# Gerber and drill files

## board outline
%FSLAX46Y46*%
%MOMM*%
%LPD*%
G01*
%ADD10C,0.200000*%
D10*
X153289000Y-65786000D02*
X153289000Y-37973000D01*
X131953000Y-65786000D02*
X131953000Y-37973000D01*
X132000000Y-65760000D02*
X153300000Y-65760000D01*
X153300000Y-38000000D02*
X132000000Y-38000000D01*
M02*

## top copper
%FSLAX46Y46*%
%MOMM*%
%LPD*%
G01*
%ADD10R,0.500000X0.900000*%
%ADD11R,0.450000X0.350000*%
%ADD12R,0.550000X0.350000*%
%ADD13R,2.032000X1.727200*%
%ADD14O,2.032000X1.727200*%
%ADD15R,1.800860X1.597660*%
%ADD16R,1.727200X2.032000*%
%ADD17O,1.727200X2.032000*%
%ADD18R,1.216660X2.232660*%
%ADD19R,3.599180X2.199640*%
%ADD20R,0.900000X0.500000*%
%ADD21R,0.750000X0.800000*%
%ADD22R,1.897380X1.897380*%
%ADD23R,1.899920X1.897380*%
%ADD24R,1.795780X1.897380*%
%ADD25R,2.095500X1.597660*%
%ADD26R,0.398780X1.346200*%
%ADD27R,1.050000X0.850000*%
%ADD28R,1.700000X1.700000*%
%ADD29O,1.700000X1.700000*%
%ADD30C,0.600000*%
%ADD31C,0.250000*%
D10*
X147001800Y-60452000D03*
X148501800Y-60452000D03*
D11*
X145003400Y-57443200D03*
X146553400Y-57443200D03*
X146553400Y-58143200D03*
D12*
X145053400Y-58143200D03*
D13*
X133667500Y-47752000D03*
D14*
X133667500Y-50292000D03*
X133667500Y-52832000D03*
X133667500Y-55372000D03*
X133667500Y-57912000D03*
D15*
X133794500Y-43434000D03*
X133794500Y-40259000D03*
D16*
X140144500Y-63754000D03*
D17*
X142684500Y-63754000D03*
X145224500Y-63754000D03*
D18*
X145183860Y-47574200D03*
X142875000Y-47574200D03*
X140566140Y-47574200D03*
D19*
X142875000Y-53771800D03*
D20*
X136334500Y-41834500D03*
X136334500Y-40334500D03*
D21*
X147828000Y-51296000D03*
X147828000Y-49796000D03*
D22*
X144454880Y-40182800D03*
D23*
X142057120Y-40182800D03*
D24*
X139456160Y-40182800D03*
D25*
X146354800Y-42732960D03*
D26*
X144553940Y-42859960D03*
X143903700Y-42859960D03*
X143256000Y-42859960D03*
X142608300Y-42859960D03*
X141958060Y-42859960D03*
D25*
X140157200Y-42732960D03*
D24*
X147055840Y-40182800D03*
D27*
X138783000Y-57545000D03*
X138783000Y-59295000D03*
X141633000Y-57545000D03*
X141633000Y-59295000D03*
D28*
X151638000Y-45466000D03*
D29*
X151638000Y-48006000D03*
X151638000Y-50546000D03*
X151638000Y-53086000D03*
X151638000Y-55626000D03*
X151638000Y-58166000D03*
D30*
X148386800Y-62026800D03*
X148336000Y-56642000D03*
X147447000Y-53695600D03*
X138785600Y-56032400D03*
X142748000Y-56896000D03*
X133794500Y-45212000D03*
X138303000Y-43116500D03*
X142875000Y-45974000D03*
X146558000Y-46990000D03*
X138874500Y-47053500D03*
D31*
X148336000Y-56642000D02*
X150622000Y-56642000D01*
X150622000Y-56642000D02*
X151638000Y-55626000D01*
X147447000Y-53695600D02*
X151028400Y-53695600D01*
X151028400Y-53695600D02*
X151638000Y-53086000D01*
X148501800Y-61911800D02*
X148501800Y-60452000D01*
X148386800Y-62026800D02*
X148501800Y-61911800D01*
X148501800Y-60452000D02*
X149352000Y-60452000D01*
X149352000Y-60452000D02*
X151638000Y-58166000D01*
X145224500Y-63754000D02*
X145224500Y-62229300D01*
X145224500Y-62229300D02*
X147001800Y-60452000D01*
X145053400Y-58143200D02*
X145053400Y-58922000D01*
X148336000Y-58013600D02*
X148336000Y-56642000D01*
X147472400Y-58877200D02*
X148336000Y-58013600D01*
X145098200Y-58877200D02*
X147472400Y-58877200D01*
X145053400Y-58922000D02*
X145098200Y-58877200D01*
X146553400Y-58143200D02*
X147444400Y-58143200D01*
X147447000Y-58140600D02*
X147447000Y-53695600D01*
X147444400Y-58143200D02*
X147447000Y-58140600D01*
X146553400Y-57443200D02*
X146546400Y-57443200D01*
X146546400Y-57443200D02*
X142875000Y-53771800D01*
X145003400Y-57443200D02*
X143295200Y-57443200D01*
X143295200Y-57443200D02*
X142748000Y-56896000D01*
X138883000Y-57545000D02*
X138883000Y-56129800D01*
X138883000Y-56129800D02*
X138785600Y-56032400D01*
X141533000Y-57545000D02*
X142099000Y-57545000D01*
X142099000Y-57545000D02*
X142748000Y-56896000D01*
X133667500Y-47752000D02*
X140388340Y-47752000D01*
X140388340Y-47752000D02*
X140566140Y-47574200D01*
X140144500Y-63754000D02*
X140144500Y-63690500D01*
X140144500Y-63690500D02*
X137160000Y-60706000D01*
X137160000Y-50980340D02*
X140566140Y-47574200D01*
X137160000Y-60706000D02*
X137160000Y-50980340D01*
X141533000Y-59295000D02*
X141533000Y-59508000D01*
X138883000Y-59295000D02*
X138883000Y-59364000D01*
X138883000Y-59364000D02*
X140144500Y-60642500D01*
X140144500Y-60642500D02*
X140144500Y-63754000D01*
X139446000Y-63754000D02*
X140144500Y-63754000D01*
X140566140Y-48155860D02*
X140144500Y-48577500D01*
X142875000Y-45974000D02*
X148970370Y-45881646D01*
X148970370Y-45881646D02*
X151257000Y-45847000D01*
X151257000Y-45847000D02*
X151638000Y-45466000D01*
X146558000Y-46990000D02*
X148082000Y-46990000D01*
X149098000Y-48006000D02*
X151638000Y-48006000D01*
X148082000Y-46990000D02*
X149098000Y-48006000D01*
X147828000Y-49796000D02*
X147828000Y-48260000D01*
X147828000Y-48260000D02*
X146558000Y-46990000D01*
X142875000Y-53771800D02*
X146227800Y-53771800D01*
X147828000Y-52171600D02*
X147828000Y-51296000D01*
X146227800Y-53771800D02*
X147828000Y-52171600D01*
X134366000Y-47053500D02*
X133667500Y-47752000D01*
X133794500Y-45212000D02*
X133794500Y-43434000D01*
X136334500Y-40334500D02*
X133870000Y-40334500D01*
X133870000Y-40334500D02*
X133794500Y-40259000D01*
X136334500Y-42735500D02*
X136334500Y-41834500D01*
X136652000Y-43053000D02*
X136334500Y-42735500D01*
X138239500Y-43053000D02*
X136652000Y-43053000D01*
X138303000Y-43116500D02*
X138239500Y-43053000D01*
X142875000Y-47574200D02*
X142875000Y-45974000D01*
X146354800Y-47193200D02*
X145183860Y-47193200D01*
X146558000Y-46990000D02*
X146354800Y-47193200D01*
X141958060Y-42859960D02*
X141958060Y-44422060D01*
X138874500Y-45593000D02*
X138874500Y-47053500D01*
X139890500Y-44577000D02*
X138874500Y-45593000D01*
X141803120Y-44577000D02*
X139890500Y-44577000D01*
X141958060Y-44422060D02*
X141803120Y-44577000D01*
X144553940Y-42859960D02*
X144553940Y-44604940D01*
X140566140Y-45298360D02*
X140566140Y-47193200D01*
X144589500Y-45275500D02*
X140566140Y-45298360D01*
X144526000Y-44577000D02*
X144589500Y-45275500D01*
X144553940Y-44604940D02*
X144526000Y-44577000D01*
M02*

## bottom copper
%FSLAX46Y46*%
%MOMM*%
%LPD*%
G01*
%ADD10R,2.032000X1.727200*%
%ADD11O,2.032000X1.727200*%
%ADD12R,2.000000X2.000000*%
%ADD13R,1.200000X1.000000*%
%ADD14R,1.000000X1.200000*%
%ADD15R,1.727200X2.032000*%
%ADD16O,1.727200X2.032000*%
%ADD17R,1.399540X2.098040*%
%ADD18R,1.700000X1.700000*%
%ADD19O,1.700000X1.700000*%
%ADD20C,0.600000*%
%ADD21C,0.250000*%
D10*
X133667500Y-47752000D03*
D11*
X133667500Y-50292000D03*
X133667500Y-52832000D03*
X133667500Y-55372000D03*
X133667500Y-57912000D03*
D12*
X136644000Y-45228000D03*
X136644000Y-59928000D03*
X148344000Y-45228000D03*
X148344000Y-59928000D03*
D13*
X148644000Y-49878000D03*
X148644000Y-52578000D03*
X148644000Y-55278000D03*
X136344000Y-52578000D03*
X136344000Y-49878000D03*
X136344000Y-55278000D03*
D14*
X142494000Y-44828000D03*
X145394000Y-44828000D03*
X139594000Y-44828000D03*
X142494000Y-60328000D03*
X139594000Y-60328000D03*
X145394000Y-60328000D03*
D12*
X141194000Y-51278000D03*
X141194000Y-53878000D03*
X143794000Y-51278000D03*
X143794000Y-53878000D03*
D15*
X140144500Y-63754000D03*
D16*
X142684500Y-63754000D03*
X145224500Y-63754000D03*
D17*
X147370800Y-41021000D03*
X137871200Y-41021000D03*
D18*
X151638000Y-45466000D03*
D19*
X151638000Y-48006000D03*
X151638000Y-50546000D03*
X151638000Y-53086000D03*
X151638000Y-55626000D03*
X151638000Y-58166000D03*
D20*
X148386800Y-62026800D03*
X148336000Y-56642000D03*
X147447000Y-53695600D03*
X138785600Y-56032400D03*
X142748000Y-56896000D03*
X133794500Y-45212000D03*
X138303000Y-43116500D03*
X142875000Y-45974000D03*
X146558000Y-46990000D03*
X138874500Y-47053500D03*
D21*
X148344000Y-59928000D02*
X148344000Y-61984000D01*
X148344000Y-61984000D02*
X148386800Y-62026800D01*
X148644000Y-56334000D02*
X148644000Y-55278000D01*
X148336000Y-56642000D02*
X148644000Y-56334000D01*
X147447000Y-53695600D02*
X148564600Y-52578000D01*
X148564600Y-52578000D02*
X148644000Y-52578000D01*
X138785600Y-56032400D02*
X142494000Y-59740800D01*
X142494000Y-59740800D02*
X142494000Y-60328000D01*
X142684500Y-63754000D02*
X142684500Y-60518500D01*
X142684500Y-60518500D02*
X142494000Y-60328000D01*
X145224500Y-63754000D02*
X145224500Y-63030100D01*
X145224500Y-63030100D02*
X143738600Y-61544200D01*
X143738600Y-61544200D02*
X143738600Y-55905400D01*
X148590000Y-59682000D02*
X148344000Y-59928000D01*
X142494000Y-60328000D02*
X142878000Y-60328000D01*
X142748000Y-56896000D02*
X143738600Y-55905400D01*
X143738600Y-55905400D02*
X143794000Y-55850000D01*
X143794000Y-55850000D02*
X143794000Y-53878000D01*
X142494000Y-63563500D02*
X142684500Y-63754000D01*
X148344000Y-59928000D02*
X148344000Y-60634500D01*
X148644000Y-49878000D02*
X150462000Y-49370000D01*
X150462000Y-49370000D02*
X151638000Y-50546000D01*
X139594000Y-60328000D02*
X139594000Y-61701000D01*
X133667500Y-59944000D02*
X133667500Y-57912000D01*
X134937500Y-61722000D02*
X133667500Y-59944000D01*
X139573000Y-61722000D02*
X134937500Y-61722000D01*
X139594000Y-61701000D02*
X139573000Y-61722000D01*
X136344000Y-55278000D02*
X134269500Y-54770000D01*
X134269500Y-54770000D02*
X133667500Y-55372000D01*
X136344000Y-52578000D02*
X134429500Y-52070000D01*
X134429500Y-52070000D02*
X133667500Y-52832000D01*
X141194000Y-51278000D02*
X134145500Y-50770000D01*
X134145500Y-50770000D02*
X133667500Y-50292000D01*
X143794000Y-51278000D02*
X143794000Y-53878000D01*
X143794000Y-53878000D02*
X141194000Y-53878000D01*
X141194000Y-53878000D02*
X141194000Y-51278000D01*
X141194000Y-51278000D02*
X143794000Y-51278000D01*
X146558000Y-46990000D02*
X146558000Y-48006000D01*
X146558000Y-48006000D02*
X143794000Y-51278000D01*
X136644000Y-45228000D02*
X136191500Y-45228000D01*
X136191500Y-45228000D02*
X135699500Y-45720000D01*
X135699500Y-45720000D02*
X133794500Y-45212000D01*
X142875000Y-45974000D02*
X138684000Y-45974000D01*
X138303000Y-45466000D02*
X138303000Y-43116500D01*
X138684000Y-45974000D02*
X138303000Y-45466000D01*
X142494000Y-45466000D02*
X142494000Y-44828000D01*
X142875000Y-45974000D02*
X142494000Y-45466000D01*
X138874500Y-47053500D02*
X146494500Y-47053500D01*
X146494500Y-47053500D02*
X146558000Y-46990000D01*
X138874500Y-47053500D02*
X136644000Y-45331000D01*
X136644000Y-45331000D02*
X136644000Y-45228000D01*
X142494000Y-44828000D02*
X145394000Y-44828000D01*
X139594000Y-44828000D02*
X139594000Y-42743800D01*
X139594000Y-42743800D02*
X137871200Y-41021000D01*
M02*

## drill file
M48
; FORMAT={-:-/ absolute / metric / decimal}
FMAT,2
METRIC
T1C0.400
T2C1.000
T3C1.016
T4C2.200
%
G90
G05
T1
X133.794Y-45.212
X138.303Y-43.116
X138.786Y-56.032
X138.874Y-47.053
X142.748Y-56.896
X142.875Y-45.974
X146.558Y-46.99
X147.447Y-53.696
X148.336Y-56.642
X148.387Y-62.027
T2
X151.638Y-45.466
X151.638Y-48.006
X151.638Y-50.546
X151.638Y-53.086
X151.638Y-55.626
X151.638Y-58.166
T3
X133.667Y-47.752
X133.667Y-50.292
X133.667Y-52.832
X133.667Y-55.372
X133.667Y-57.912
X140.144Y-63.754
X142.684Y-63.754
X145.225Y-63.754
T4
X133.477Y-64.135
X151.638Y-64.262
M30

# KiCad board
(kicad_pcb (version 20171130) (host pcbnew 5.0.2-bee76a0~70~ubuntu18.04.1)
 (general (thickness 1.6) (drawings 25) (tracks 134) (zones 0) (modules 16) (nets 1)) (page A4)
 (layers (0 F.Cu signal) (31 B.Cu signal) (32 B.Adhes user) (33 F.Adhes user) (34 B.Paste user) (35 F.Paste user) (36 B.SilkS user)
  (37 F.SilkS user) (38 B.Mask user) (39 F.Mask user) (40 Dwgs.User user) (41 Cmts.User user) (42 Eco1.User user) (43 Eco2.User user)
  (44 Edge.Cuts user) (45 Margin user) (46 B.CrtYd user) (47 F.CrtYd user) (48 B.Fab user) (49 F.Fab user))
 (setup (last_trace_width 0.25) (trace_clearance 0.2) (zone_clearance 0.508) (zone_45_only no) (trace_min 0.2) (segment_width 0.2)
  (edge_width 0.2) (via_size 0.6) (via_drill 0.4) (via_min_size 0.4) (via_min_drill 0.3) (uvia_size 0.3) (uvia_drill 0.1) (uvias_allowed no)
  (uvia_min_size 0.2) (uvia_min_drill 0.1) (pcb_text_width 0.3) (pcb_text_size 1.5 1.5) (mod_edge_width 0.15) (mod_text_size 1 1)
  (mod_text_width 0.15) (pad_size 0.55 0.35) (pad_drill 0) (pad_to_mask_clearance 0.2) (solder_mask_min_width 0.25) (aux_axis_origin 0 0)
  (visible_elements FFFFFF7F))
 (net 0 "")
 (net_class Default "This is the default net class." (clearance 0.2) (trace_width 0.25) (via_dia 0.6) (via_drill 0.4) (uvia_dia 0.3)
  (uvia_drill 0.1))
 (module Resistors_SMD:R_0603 (layer F.Cu) (at 147.7518 60.452)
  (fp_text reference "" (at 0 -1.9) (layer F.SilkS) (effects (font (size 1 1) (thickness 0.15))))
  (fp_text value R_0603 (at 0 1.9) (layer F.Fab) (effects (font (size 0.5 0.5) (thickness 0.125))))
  (pad 1 smd rect (at -0.75 0) (size 0.5 0.9) (layers F.Cu F.Paste F.Mask))
  (pad 2 smd rect (at 0.75 0) (size 0.5 0.9) (layers F.Cu F.Paste F.Mask)))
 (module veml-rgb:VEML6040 (layer F.Cu) (at 145.9484 56.7182)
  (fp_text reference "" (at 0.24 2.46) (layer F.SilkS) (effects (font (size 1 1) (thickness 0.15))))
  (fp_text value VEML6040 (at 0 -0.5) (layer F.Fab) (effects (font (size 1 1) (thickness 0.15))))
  (pad GND smd rect (at -0.945 0.725) (size 0.45 0.35) (layers F.Cu F.Paste F.Mask))
  (pad +V smd rect (at 0.605 0.725) (size 0.45 0.35) (layers F.Cu F.Paste F.Mask))
  (pad 3 smd rect (at 0.605 1.425) (size 0.45 0.35) (layers F.Cu F.Paste F.Mask))
  (pad 2 smd rect (at -0.895 1.425) (size 0.55 0.35) (layers F.Cu F.Paste F.Mask)))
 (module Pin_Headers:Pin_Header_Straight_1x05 (layer F.Cu) (at 133.6675 47.752)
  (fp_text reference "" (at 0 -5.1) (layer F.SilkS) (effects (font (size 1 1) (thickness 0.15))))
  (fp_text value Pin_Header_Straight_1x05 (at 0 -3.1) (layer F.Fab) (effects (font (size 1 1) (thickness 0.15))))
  (pad 1 thru_hole rect (at 0 0) (size 2.032 1.7272) (drill 1.016) (layers *.Cu *.Mask F.SilkS))
  (pad 2 thru_hole oval (at 0 2.54) (size 2.032 1.7272) (drill 1.016) (layers *.Cu *.Mask F.SilkS))
  (pad 3 thru_hole oval (at 0 5.08) (size 2.032 1.7272) (drill 1.016) (layers *.Cu *.Mask F.SilkS))
  (pad 4 thru_hole oval (at 0 7.62) (size 2.032 1.7272) (drill 1.016) (layers *.Cu *.Mask F.SilkS))
  (pad 5 thru_hole oval (at 0 10.16) (size 2.032 1.7272) (drill 1.016) (layers *.Cu *.Mask F.SilkS)))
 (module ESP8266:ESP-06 (layer B.Cu) (at 142.494 52.578 270)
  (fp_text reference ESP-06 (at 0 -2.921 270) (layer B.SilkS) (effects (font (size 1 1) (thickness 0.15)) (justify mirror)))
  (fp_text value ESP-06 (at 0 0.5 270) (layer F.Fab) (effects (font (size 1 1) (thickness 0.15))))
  (pad GND smd rect (at -7.35 5.85 270) (size 2 2) (layers B.Cu B.Paste B.Mask))
  (pad GP5 smd rect (at 7.35 5.85 270) (size 2 2) (layers B.Cu B.Paste B.Mask))
  (pad GP16 smd rect (at -7.35 -5.85 270) (size 2 2) (layers B.Cu B.Paste B.Mask))
  (pad GP15 smd rect (at 7.35 -5.85 270) (size 2 2) (layers B.Cu B.Paste B.Mask))
  (pad GP14 smd rect (at -2.7 -6.15 270) (size 1 1.2) (layers B.Cu B.Paste B.Mask))
  (pad GP12 smd rect (at 0 -6.15 270) (size 1 1.2) (layers B.Cu B.Paste B.Mask))
  (pad GP13 smd rect (at 2.7 -6.15 270) (size 1 1.2) (layers B.Cu B.Paste B.Mask))
  (pad TX smd rect (at 0 6.15 270) (size 1 1.2) (layers B.Cu B.Paste B.Mask))
  (pad RST smd rect (at -2.7 6.15 270) (size 1 1.2) (layers B.Cu B.Paste B.Mask))
  (pad RX smd rect (at 2.7 6.15 270) (size 1 1.2) (layers B.Cu B.Paste B.Mask))
  (pad 3.3 smd rect (at -7.75 0 270) (size 1.2 1) (layers B.Cu B.Paste B.Mask))
  (pad CHPD smd rect (at -7.75 -2.9 270) (size 1.2 1) (layers B.Cu B.Paste B.Mask))
  (pad ANT smd rect (at -7.75 2.9 270) (size 1.2 1) (layers B.Cu B.Paste B.Mask))
  (pad GP2 smd rect (at 7.75 0 270) (size 1.2 1) (layers B.Cu B.Paste B.Mask))
  (pad GP0 smd rect (at 7.75 2.9 270) (size 1.2 1) (layers B.Cu B.Paste B.Mask))
  (pad GP4 smd rect (at 7.75 -2.9 270) (size 1.2 1) (layers B.Cu B.Paste B.Mask))
  (pad GND smd rect (at -1.3 1.3 270) (size 2 2) (layers B.Cu B.Paste B.Mask))
  (pad GND smd rect (at 1.3 1.3 270) (size 2 2) (layers B.Cu B.Paste B.Mask))
  (pad GND smd rect (at -1.3 -1.3 270) (size 2 2) (layers B.Cu B.Paste B.Mask))
  (pad GND smd rect (at 1.3 -1.3 270) (size 2 2) (layers B.Cu B.Paste B.Mask)))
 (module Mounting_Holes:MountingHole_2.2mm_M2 (layer F.Cu) (at 133.477 64.135)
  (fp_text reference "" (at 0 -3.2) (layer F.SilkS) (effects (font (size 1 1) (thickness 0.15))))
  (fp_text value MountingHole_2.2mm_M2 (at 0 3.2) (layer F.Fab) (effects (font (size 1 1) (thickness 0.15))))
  (pad 1 np_thru_hole circle (at 0 0) (size 2.2 2.2) (drill 2.2) (layers *.Cu *.Mask F.SilkS)))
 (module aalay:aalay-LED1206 (layer F.Cu) (at 133.7945 41.8465 90)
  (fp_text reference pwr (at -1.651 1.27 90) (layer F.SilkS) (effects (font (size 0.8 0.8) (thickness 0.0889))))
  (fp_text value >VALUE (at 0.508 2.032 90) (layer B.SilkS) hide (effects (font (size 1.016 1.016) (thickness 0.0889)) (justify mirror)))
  (pad A smd rect (at -1.5875 0 90) (size 1.59766 1.80086) (layers F.Cu F.Paste F.Mask))
  (pad K smd rect (at 1.5875 0 90) (size 1.59766 1.80086) (layers F.Cu F.Paste F.Mask)))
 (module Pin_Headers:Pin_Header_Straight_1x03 (layer F.Cu) (at 140.1445 63.754 90)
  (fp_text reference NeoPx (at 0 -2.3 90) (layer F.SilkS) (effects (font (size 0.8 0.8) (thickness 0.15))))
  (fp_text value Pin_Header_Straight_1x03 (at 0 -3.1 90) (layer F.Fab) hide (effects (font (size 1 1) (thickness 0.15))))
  (pad 1 thru_hole rect (at 0 0 90) (size 2.032 1.7272) (drill 1.016) (layers *.Cu *.Mask F.SilkS))
  (pad 2 thru_hole oval (at 0 2.54 90) (size 2.032 1.7272) (drill 1.016) (layers *.Cu *.Mask F.SilkS))
  (pad 3 thru_hole oval (at 0 5.08 90) (size 2.032 1.7272) (drill 1.016) (layers *.Cu *.Mask F.SilkS)))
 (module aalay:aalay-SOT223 (layer F.Cu) (at 142.875 50.673 180)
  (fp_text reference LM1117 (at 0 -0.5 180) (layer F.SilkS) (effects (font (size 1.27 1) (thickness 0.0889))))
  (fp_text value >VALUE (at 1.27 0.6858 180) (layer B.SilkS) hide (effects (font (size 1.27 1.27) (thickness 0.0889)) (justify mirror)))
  (pad GND smd rect (at -2.30886 3.0988 180) (size 1.21666 2.23266) (layers F.Cu F.Paste F.Mask))
  (pad OUT smd rect (at 0 3.0988 180) (size 1.21666 2.23266) (layers F.Cu F.Paste F.Mask))
  (pad IN smd rect (at 2.30886 3.0988 180) (size 1.21666 2.23266) (layers F.Cu F.Paste F.Mask))
  (pad OUT smd rect (at 0 -3.0988 180) (size 3.59918 2.19964) (layers F.Cu F.Paste F.Mask)))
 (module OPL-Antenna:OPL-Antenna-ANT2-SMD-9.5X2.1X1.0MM (layer B.Cu) (at 142.621 41.021 180)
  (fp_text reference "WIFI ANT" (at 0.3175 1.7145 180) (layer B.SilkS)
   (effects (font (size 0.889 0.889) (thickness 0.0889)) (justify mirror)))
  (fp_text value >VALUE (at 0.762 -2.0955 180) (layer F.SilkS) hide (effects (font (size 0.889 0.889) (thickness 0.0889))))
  (pad 1 smd rect (at -4.7498 0 180) (size 1.39954 2.09804) (layers B.Cu B.Paste B.Mask))
  (pad 2 smd rect (at 4.7498 0 180) (size 1.39954 2.09804) (layers B.Cu B.Paste B.Mask)))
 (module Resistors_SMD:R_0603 (layer F.Cu) (at 136.3345 41.0845 90)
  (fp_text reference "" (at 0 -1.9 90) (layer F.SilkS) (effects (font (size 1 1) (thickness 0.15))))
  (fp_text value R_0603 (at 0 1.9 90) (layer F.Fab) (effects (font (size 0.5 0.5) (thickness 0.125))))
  (pad 1 smd rect (at -0.75 0 90) (size 0.5 0.9) (layers F.Cu F.Paste F.Mask))
  (pad 2 smd rect (at 0.75 0 90) (size 0.5 0.9) (layers F.Cu F.Paste F.Mask)))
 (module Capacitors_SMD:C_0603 (layer F.Cu) (at 147.828 50.546 90)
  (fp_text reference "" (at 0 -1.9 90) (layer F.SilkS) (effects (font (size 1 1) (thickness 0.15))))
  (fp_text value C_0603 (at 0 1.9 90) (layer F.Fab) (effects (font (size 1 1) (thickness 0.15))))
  (pad 1 smd rect (at -0.75 0 90) (size 0.8 0.75) (layers F.Cu F.Paste F.Mask))
  (pad 2 smd rect (at 0.75 0 90) (size 0.8 0.75) (layers F.Cu F.Paste F.Mask)))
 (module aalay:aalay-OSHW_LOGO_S (layer F.Cu) (at 150.622 39.878)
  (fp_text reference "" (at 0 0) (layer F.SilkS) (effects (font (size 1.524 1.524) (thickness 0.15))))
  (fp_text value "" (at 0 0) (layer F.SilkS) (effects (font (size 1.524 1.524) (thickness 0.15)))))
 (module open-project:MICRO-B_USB (layer F.Cu) (at 143.256 38.735 180)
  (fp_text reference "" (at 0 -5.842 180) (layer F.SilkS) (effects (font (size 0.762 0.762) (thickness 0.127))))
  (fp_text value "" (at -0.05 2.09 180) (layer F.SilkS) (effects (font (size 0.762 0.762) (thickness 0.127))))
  (pad "" smd rect (at -1.19888 -1.4478 180) (size 1.89738 1.89738) (layers F.Cu F.Paste F.Mask))
  (pad "" smd rect (at 1.19888 -1.4478 180) (size 1.89992 1.89738) (layers F.Cu F.Paste F.Mask))
  (pad "" smd rect (at 3.79984 -1.4478 180) (size 1.79578 1.89738) (layers F.Cu F.Paste F.Mask))
  (pad "" smd rect (at -3.0988 -3.99796 180) (size 2.0955 1.59766) (layers F.Cu F.Paste F.Mask))
  (pad +5 smd rect (at -1.29794 -4.12496 180) (size 0.39878 1.3462) (layers F.Cu F.Paste F.Mask) (clearance 0.2032))
  (pad 2 smd rect (at -0.6477 -4.12496 180) (size 0.39878 1.3462) (layers F.Cu F.Paste F.Mask) (clearance 0.2032))
  (pad 3 smd rect (at 0 -4.12496 180) (size 0.39878 1.3462) (layers F.Cu F.Paste F.Mask) (clearance 0.2032))
  (pad 4 smd rect (at 0.6477 -4.12496 180) (size 0.39878 1.3462) (layers F.Cu F.Paste F.Mask) (clearance 0.2032))
  (pad GND smd rect (at 1.29794 -4.12496 180) (size 0.39878 1.3462) (layers F.Cu F.Paste F.Mask) (clearance 0.2032))
  (pad "" smd rect (at 3.0988 -3.99796 180) (size 2.0955 1.59766) (layers F.Cu F.Paste F.Mask))
  (pad "" smd rect (at -3.79984 -1.4478 180) (size 1.79578 1.89738) (layers F.Cu F.Paste F.Mask)))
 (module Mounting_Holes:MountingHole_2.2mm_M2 (layer F.Cu) (at 151.638 64.262)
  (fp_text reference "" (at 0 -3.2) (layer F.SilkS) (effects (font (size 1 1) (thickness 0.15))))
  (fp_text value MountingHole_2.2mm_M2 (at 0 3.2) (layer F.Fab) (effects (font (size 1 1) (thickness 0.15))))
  (pad 1 np_thru_hole circle (at 0 0) (size 2.2 2.2) (drill 2.2) (layers *.Cu *.Mask F.SilkS)))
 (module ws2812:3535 (layer F.Cu) (at 140.208 58.42 180)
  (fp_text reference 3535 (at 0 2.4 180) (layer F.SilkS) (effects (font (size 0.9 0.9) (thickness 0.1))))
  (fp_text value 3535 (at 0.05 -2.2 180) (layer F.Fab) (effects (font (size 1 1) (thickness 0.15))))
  (pad IN smd rect (at 1.325 0.875 180) (size 1.05 0.85) (drill (offset 0.1 0)) (layers F.Cu F.Paste F.Mask))
  (pad VDD smd rect (at 1.325 -0.875 180) (size 1.05 0.85) (drill (offset 0.1 0)) (layers F.Cu F.Paste F.Mask))
  (pad GND smd rect (at -1.325 0.875 180) (size 1.05 0.85) (drill (offset -0.1 0)) (layers F.Cu F.Paste F.Mask))
  (pad OUT smd rect (at -1.325 -0.875 180) (size 1.05 0.85) (drill (offset -0.1 0)) (layers F.Cu F.Paste F.Mask)))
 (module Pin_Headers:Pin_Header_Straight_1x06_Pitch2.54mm (layer F.Cu) (at 151.638 45.466)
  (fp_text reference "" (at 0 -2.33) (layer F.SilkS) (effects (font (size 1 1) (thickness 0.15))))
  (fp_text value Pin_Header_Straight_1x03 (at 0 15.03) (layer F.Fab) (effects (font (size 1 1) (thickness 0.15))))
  (pad 1 thru_hole rect (at 0 0) (size 1.7 1.7) (drill 1) (layers *.Cu *.Mask))
  (pad 2 thru_hole oval (at 0 2.54) (size 1.7 1.7) (drill 1) (layers *.Cu *.Mask))
  (pad 3 thru_hole oval (at 0 5.08) (size 1.7 1.7) (drill 1) (layers *.Cu *.Mask))
  (pad 4 thru_hole oval (at 0 7.62) (size 1.7 1.7) (drill 1) (layers *.Cu *.Mask))
  (pad 5 thru_hole oval (at 0 10.16) (size 1.7 1.7) (drill 1) (layers *.Cu *.Mask))
  (pad 6 thru_hole oval (at 0 12.7) (size 1.7 1.7) (drill 1) (layers *.Cu *.Mask)))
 (gr_line (start 153.289 65.786) (end 153.289 37.973) (angle 90) (layer Edge.Cuts) (width 0.2))
 (gr_line (start 131.953 65.786) (end 131.953 37.973) (angle 90) (layer Edge.Cuts) (width 0.2))
 (gr_line (start 132 65.76) (end 153.3 65.76) (angle 90) (layer Edge.Cuts) (width 0.2))
 (gr_line (start 153.3 38) (end 132 38) (angle 90) (layer Edge.Cuts) (width 0.2))
 (segment (start 148.336 56.642) (end 150.622 56.642) (width 0.25) (layer F.Cu) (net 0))
 (segment (start 150.622 56.642) (end 151.638 55.626) (width 0.25) (layer F.Cu) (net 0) (status 800000))
 (segment (start 147.447 53.6956) (end 151.0284 53.6956) (width 0.25) (layer F.Cu) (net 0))
 (segment (start 151.0284 53.6956) (end 151.638 53.086) (width 0.25) (layer F.Cu) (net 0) (status 800000))
 (segment (start 148.344 59.928) (end 148.344 61.984) (width 0.25) (layer B.Cu) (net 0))
 (segment (start 148.5018 61.9118) (end 148.5018 60.452) (width 0.25) (layer F.Cu) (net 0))
 (segment (start 148.3868 62.0268) (end 148.5018 61.9118) (width 0.25) (layer F.Cu) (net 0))
 (via (at 148.3868 62.0268) (size 0.6) (drill 0.4) (layers F.Cu B.Cu) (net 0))
 (segment (start 148.344 61.984) (end 148.3868 62.0268) (width 0.25) (layer B.Cu) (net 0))
 (segment (start 148.5018 60.452) (end 149.352 60.452) (width 0.25) (layer F.Cu) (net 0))
 (segment (start 149.352 60.452) (end 151.638 58.166) (width 0.25) (layer F.Cu) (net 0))
 (segment (start 145.2245 63.754) (end 145.2245 62.2293) (width 0.25) (layer F.Cu) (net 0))
 (segment (start 145.2245 62.2293) (end 147.0018 60.452) (width 0.25) (layer F.Cu) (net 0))
 (segment (start 145.0534 58.1432) (end 145.0534 58.922) (width 0.25) (layer F.Cu) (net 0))
 (segment (start 148.644 56.334) (end 148.644 55.278) (width 0.25) (layer B.Cu) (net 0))
 (segment (start 148.336 56.642) (end 148.644 56.334) (width 0.25) (layer B.Cu) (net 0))
 (via (at 148.336 56.642) (size 0.6) (drill 0.4) (layers F.Cu B.Cu) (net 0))
 (segment (start 148.336 58.0136) (end 148.336 56.642) (width 0.25) (layer F.Cu) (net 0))
 (segment (start 147.4724 58.8772) (end 148.336 58.0136) (width 0.25) (layer F.Cu) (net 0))
 (segment (start 145.0982 58.8772) (end 147.4724 58.8772) (width 0.25) (layer F.Cu) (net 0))
 (segment (start 145.0534 58.922) (end 145.0982 58.8772) (width 0.25) (layer F.Cu) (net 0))
 (segment (start 146.5534 58.1432) (end 147.4444 58.1432) (width 0.25) (layer F.Cu) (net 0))
 (segment (start 147.447 53.6956) (end 148.5646 52.578) (width 0.25) (layer B.Cu) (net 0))
 (via (at 147.447 53.6956) (size 0.6) (drill 0.4) (layers F.Cu B.Cu) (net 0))
 (segment (start 147.447 58.1406) (end 147.447 53.6956) (width 0.25) (layer F.Cu) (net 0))
 (segment (start 147.4444 58.1432) (end 147.447 58.1406) (width 0.25) (layer F.Cu) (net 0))
 (segment (start 148.5646 52.578) (end 148.644 52.578) (width 0.25) (layer B.Cu) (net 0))
 (segment (start 146.5534 57.4432) (end 146.5464 57.4432) (width 0.25) (layer F.Cu) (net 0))
 (segment (start 146.5464 57.4432) (end 142.875 53.7718) (width 0.25) (layer F.Cu) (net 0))
 (segment (start 145.0034 57.4432) (end 143.2952 57.4432) (width 0.25) (layer F.Cu) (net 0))
 (segment (start 143.2952 57.4432) (end 142.748 56.896) (width 0.25) (layer F.Cu) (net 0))
 (segment (start 138.883 57.545) (end 138.883 56.1298) (width 0.25) (layer F.Cu) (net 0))
 (segment (start 138.7856 56.0324) (end 142.494 59.7408) (width 0.25) (layer B.Cu) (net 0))
 (via (at 138.7856 56.0324) (size 0.6) (drill 0.4) (layers F.Cu B.Cu) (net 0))
 (segment (start 138.883 56.1298) (end 138.7856 56.0324) (width 0.25) (layer F.Cu) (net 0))
 (segment (start 142.494 59.7408) (end 142.494 60.328) (width 0.25) (layer B.Cu) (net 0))
 (segment (start 142.6845 63.754) (end 142.6845 60.5185) (width 0.25) (layer B.Cu) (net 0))
 (segment (start 142.6845 60.5185) (end 142.494 60.328) (width 0.25) (layer B.Cu) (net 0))
 (segment (start 145.2245 63.754) (end 145.2245 63.0301) (width 0.25) (layer B.Cu) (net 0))
 (segment (start 145.2245 63.0301) (end 143.7386 61.5442) (width 0.25) (layer B.Cu) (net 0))
 (segment (start 143.7386 61.5442) (end 143.7386 55.9054) (width 0.25) (layer B.Cu) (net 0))
 (segment (start 148.59 59.682) (end 148.344 59.928) (width 0.25) (layer B.Cu) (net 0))
 (segment (start 142.494 60.328) (end 142.878 60.328) (width 0.25) (layer B.Cu) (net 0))
 (segment (start 141.533 57.545) (end 142.099 57.545) (width 0.25) (layer F.Cu) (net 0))
 (segment (start 142.099 57.545) (end 142.748 56.896) (width 0.25) (layer F.Cu) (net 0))
 (via (at 142.748 56.896) (size 0.6) (drill 0.4) (layers F.Cu B.Cu) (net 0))
 (segment (start 142.748 56.896) (end 143.7386 55.9054) (width 0.25) (layer B.Cu) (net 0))
 (segment (start 143.7386 55.9054) (end 143.794 55.85) (width 0.25) (layer B.Cu) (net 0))
 (segment (start 143.794 55.85) (end 143.794 53.878) (width 0.25) (layer B.Cu) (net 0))
 (segment (start 133.6675 47.752) (end 140.38834 47.752) (width 0.25) (layer F.Cu) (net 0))
 (segment (start 140.38834 47.752) (end 140.56614 47.5742) (width 0.25) (layer F.Cu) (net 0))
 (segment (start 140.1445 63.754) (end 140.1445 63.6905) (width 0.25) (layer F.Cu) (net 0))
 (segment (start 140.1445 63.6905) (end 137.16 60.706) (width 0.25) (layer F.Cu) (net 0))
 (segment (start 137.16 50.98034) (end 140.56614 47.5742) (width 0.25) (layer F.Cu) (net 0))
 (segment (start 137.16 60.706) (end 137.16 50.98034) (width 0.25) (layer F.Cu) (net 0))
 (segment (start 142.494 63.5635) (end 142.6845 63.754) (width 0.25) (layer B.Cu) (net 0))
 (segment (start 141.533 59.295) (end 141.533 59.508) (width 0.25) (layer F.Cu) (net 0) (status 30))
 (segment (start 138.883 59.295) (end 138.883 59.364) (width 0.25) (layer F.Cu) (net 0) (status 30))
 (segment (start 138.883 59.364) (end 140.1445 60.6425) (width 0.25) (layer F.Cu) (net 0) (status 10))
 (segment (start 140.1445 60.6425) (end 140.1445 63.754) (width 0.25) (layer F.Cu) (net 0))
 (segment (start 139.446 63.754) (end 140.1445 63.754) (width 0.25) (layer F.Cu) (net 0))
 (segment (start 140.56614 48.15586) (end 140.1445 48.5775) (width 0.25) (layer F.Cu) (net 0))
 (segment (start 148.344 59.928) (end 148.344 60.6345) (width 0.25) (layer B.Cu) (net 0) (status 10))
 (segment (start 148.644 49.878) (end 150.462 49.37) (width 0.25) (layer B.Cu) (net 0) (status 10))
 (segment (start 150.462 49.37) (end 151.638 50.546) (width 0.25) (layer B.Cu) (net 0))
 (segment (start 142.875 45.974) (end 148.97037 45.881646) (width 0.25) (layer F.Cu) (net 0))
 (segment (start 148.97037 45.881646) (end 151.257 45.847) (width 0.25) (layer F.Cu) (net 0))
 (segment (start 151.257 45.847) (end 151.638 45.466) (width 0.25) (layer F.Cu) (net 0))
 (segment (start 146.558 46.99) (end 148.082 46.99) (width 0.25) (layer F.Cu) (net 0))
 (segment (start 149.098 48.006) (end 151.638 48.006) (width 0.25) (layer F.Cu) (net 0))
 (segment (start 148.082 46.99) (end 149.098 48.006) (width 0.25) (layer F.Cu) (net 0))
 (segment (start 147.828 49.796) (end 147.828 48.26) (width 0.25) (layer F.Cu) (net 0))
 (segment (start 147.828 48.26) (end 146.558 46.99) (width 0.25) (layer F.Cu) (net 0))
 (segment (start 142.875 53.7718) (end 146.2278 53.7718) (width 0.25) (layer F.Cu) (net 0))
 (segment (start 147.828 52.1716) (end 147.828 51.296) (width 0.25) (layer F.Cu) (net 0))
 (segment (start 146.2278 53.7718) (end 147.828 52.1716) (width 0.25) (layer F.Cu) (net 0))
 (segment (start 139.594 60.328) (end 139.594 61.701) (width 0.25) (layer B.Cu) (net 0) (status 10))
 (segment (start 133.6675 59.944) (end 133.6675 57.912) (width 0.25) (layer B.Cu) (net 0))
 (segment (start 134.9375 61.722) (end 133.6675 59.944) (width 0.25) (layer B.Cu) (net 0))
 (segment (start 139.573 61.722) (end 134.9375 61.722) (width 0.25) (layer B.Cu) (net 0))
 (segment (start 139.594 61.701) (end 139.573 61.722) (width 0.25) (layer B.Cu) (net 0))
 (segment (start 136.344 55.278) (end 134.2695 54.77) (width 0.25) (layer B.Cu) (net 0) (status 10))
 (segment (start 134.2695 54.77) (end 133.6675 55.372) (width 0.25) (layer B.Cu) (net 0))
 (segment (start 136.344 52.578) (end 134.4295 52.07) (width 0.25) (layer B.Cu) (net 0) (status 10))
 (segment (start 134.4295 52.07) (end 133.6675 52.832) (width 0.25) (layer B.Cu) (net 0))
 (segment (start 141.194 51.278) (end 134.1455 50.77) (width 0.25) (layer B.Cu) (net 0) (status 10))
 (segment (start 134.1455 50.77) (end 133.6675 50.292) (width 0.25) (layer B.Cu) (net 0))
 (segment (start 134.366 47.0535) (end 133.6675 47.752) (width 0.25) (layer F.Cu) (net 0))
 (segment (start 143.794 51.278) (end 143.794 53.878) (width 0.25) (layer B.Cu) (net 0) (status 30))
 (segment (start 143.794 53.878) (end 141.194 53.878) (width 0.25) (layer B.Cu) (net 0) (status 30))
 (segment (start 141.194 53.878) (end 141.194 51.278) (width 0.25) (layer B.Cu) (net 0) (status 30))
 (segment (start 141.194 51.278) (end 143.794 51.278) (width 0.25) (layer B.Cu) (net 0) (status 30))
 (segment (start 146.558 46.99) (end 146.558 48.006) (width 0.25) (layer B.Cu) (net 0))
 (segment (start 146.558 48.006) (end 143.794 51.278) (width 0.25) (layer B.Cu) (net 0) (status 20))
 (segment (start 136.644 45.228) (end 136.1915 45.228) (width 0.25) (layer B.Cu) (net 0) (status 30))
 (segment (start 136.1915 45.228) (end 135.6995 45.72) (width 0.25) (layer B.Cu) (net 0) (status 30))
 (segment (start 135.6995 45.72) (end 133.7945 45.212) (width 0.25) (layer B.Cu) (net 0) (status 10))
 (via (at 133.7945 45.212) (size 0.6) (drill 0.4) (layers F.Cu B.Cu) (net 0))
 (segment (start 133.7945 45.212) (end 133.7945 43.434) (width 0.25) (layer F.Cu) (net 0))
 (segment (start 136.3345 40.3345) (end 133.87 40.3345) (width 0.25) (layer F.Cu) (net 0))
 (segment (start 133.87 40.3345) (end 133.7945 40.259) (width 0.25) (layer F.Cu) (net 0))
 (segment (start 142.875 45.974) (end 138.684 45.974) (width 0.25) (layer B.Cu) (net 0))
 (segment (start 136.3345 42.7355) (end 136.3345 41.8345) (width 0.25) (layer F.Cu) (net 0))
 (segment (start 136.652 43.053) (end 136.3345 42.7355) (width 0.25) (layer F.Cu) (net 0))
 (segment (start 138.2395 43.053) (end 136.652 43.053) (width 0.25) (layer F.Cu) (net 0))
 (segment (start 138.303 43.1165) (end 138.2395 43.053) (width 0.25) (layer F.Cu) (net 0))
 (via (at 138.303 43.1165) (size 0.6) (drill 0.4) (layers F.Cu B.Cu) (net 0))
 (segment (start 138.303 45.466) (end 138.303 43.1165) (width 0.25) (layer B.Cu) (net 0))
 (segment (start 138.684 45.974) (end 138.303 45.466) (width 0.25) (layer B.Cu) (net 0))
 (segment (start 142.875 47.5742) (end 142.875 45.974) (width 0.25) (layer F.Cu) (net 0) (status 10))
 (segment (start 142.494 45.466) (end 142.494 44.828) (width 0.25) (layer B.Cu) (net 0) (status 20))
 (segment (start 142.875 45.974) (end 142.494 45.466) (width 0.25) (layer B.Cu) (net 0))
 (via (at 142.875 45.974) (size 0.6) (drill 0.4) (layers F.Cu B.Cu) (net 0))
 (segment (start 138.8745 47.0535) (end 146.4945 47.0535) (width 0.25) (layer B.Cu) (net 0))
 (segment (start 146.3548 47.1932) (end 145.18386 47.1932) (width 0.25) (layer F.Cu) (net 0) (status 20))
 (segment (start 146.558 46.99) (end 146.3548 47.1932) (width 0.25) (layer F.Cu) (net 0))
 (via (at 146.558 46.99) (size 0.6) (drill 0.4) (layers F.Cu B.Cu) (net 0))
 (segment (start 146.4945 47.0535) (end 146.558 46.99) (width 0.25) (layer B.Cu) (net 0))
 (segment (start 141.95806 42.85996) (end 141.95806 44.42206) (width 0.25) (layer F.Cu) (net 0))
 (segment (start 138.8745 47.0535) (end 136.644 45.331) (width 0.25) (layer B.Cu) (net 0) (status 20))
 (via (at 138.8745 47.0535) (size 0.6) (drill 0.4) (layers F.Cu B.Cu) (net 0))
 (segment (start 138.8745 45.593) (end 138.8745 47.0535) (width 0.25) (layer F.Cu) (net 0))
 (segment (start 139.8905 44.577) (end 138.8745 45.593) (width 0.25) (layer F.Cu) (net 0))
 (segment (start 141.80312 44.577) (end 139.8905 44.577) (width 0.25) (layer F.Cu) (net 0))
 (segment (start 141.95806 44.42206) (end 141.80312 44.577) (width 0.25) (layer F.Cu) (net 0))
 (segment (start 136.644 45.331) (end 136.644 45.228) (width 0.25) (layer B.Cu) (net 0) (status 30))
 (segment (start 144.55394 42.85996) (end 144.55394 44.60494) (width 0.25) (layer F.Cu) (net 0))
 (segment (start 140.56614 45.29836) (end 140.56614 47.1932) (width 0.25) (layer F.Cu) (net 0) (status 20))
 (segment (start 144.5895 45.2755) (end 140.56614 45.29836) (width 0.25) (layer F.Cu) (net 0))
 (segment (start 144.526 44.577) (end 144.5895 45.2755) (width 0.25) (layer F.Cu) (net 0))
 (segment (start 144.55394 44.60494) (end 144.526 44.577) (width 0.25) (layer F.Cu) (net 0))
 (segment (start 142.494 44.828) (end 145.394 44.828) (width 0.25) (layer B.Cu) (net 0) (status 30))
 (segment (start 139.594 44.828) (end 139.594 42.7438) (width 0.25) (layer B.Cu) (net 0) (status 10))
 (segment (start 139.594 42.7438) (end 137.8712 41.021) (width 0.25) (layer B.Cu) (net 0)))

